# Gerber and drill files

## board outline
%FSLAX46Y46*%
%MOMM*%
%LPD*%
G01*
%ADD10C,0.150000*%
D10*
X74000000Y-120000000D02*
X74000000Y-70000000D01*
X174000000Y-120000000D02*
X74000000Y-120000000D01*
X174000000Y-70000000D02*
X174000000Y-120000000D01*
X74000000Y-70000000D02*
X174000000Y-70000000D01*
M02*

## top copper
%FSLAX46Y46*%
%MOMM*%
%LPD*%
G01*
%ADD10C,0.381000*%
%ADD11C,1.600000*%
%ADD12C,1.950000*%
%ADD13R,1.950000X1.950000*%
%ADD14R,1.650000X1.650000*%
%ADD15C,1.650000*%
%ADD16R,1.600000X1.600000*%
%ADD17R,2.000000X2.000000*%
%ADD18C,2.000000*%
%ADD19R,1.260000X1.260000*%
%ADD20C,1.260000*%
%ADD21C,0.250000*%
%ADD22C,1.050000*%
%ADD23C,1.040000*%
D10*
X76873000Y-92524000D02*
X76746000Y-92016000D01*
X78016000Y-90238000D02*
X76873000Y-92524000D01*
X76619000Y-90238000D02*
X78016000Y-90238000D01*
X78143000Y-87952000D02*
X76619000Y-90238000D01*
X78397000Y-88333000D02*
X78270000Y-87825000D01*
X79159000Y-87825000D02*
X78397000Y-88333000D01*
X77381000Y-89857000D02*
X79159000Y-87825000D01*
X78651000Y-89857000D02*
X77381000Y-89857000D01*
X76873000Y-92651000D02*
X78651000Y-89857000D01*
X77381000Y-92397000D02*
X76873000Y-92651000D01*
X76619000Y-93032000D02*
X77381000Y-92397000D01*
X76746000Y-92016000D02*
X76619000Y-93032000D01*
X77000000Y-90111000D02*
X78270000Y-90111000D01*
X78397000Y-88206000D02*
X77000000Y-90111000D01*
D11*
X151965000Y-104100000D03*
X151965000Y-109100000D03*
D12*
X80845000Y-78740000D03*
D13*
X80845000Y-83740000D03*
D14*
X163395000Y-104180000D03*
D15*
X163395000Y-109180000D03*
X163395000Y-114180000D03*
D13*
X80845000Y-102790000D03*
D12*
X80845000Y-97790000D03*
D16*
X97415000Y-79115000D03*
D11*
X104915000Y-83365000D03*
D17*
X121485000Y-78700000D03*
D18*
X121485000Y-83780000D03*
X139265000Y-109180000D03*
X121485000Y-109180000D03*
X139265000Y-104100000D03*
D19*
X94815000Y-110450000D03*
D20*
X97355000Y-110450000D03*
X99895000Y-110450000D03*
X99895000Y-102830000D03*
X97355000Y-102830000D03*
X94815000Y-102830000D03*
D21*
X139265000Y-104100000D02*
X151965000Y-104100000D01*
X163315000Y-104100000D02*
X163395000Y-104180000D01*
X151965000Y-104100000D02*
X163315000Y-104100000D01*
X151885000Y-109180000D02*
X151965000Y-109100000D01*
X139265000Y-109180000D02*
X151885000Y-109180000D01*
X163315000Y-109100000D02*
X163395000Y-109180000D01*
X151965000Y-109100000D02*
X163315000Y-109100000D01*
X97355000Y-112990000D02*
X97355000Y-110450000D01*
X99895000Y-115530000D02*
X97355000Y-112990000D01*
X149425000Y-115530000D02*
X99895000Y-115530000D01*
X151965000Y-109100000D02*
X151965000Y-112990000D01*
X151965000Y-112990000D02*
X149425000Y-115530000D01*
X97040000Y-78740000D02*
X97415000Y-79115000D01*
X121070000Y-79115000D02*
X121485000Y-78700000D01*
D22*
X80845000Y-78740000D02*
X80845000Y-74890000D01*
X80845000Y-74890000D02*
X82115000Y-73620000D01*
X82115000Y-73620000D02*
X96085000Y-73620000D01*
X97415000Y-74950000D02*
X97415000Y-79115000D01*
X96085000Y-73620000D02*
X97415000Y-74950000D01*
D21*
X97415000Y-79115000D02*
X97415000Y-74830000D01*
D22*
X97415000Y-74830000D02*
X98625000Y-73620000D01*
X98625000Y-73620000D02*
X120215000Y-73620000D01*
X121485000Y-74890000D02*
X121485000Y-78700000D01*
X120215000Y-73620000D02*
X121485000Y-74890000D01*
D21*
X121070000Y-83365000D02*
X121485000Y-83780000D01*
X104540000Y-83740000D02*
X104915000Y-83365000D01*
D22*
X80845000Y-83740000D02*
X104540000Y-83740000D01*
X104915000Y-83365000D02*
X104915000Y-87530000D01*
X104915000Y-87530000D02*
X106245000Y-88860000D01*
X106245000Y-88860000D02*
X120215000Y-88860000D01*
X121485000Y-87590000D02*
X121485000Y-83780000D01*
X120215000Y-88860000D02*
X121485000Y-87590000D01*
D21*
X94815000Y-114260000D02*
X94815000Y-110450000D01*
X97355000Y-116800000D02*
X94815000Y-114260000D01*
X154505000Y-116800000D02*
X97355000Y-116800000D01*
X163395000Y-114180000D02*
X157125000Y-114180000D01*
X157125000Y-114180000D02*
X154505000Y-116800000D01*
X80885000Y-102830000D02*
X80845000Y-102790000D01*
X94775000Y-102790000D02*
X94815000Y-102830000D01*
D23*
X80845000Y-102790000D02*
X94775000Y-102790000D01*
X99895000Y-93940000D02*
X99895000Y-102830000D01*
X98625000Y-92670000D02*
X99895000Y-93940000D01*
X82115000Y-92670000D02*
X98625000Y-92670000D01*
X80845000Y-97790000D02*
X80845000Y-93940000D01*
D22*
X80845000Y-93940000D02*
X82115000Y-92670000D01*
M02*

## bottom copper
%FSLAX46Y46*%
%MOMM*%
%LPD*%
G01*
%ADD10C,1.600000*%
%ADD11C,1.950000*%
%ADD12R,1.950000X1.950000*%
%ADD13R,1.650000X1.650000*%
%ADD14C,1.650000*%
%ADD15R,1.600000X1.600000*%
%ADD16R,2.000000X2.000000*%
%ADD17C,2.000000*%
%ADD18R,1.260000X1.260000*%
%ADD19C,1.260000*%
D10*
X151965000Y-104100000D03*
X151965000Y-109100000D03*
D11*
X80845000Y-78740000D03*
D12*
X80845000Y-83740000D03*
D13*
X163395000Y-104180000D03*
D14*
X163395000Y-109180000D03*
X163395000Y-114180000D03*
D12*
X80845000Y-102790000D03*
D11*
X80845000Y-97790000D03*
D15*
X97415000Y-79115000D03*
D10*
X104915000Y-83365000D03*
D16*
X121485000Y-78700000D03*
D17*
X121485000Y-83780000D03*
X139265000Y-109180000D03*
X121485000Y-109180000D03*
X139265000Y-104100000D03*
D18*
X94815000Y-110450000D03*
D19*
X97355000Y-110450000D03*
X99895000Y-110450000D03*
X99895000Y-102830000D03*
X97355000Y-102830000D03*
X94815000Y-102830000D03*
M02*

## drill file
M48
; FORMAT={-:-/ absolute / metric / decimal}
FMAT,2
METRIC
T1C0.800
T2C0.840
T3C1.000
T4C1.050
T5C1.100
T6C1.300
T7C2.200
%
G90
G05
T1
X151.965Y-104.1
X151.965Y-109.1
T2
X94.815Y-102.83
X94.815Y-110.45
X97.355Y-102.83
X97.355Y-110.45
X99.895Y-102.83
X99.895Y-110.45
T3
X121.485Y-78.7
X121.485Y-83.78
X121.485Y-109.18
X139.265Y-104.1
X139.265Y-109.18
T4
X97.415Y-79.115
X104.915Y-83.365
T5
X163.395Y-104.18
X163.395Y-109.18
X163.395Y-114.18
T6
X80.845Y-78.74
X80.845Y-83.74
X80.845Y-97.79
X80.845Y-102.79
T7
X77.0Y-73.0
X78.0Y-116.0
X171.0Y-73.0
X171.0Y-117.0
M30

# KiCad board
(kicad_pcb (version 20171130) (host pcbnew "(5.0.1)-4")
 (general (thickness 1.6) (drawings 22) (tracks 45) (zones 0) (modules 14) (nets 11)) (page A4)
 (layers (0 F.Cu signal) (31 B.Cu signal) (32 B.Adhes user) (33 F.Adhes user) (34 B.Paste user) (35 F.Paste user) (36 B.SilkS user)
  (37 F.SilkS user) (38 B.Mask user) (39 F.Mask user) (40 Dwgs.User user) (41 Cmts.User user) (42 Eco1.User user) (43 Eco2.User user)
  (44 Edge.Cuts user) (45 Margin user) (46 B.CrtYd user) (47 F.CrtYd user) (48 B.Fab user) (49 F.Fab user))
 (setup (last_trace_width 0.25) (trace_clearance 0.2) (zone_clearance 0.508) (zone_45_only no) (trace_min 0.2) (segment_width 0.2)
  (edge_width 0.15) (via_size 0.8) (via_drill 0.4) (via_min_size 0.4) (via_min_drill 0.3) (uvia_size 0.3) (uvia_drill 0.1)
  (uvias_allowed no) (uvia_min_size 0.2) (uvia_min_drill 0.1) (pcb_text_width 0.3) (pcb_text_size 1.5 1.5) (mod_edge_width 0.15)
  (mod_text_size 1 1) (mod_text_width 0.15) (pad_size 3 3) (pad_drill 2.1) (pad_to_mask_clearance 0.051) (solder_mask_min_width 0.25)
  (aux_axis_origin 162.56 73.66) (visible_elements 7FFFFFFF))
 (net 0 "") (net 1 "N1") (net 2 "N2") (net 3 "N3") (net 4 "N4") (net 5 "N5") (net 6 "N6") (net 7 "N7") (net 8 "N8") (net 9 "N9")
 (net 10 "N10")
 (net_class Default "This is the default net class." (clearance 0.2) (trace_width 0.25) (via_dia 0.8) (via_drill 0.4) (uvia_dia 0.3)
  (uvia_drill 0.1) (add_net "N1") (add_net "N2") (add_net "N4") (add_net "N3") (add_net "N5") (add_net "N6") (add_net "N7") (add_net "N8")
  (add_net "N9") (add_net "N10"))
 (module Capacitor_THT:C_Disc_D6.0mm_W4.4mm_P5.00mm (layer F.Cu) (at 151.965 104.1 270)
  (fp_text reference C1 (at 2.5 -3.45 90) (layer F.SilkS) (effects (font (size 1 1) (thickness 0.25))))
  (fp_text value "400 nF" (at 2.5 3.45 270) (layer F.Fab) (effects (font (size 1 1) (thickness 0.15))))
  (pad 1 thru_hole circle (at 0 0 270) (size 1.6 1.6) (drill 0.8) (layers *.Cu *.Mask) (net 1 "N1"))
  (pad 2 thru_hole circle (at 5 0 270) (size 1.6 1.6) (drill 0.8) (layers *.Cu *.Mask) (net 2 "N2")))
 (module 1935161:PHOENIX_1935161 (layer F.Cu) (at 80.845 81.24 90)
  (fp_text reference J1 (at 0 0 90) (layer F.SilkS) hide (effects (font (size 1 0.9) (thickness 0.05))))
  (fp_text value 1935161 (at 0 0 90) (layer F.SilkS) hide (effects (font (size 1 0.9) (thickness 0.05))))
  (pad 2 thru_hole circle (at 2.5 0 90) (size 1.95 1.95) (drill 1.3) (layers *.Cu *.Mask) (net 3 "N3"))
  (pad 1 thru_hole rect (at -2.5 0 90) (size 1.95 1.95) (drill 1.3) (layers *.Cu *.Mask) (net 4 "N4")))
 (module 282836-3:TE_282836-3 (layer F.Cu) (at 163.395 109.18 270)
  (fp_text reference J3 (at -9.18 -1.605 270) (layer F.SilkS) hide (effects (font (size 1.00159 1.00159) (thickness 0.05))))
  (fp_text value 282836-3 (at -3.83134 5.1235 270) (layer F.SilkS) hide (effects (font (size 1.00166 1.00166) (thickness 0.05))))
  (pad 1 thru_hole rect (at -5 0 270) (size 1.65 1.65) (drill 1.1) (layers *.Cu *.Mask) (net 1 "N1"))
  (pad 2 thru_hole circle (at 0 0 270) (size 1.65 1.65) (drill 1.1) (layers *.Cu *.Mask) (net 2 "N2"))
  (pad 3 thru_hole circle (at 5 0 270) (size 1.65 1.65) (drill 1.1) (layers *.Cu *.Mask) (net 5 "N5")))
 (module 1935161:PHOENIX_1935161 (layer F.Cu) (at 80.845 100.29 90)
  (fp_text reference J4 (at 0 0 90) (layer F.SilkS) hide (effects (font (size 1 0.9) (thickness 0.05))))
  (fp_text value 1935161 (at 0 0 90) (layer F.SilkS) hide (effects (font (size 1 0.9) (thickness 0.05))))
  (pad 1 thru_hole rect (at -2.5 0 90) (size 1.95 1.95) (drill 1.3) (layers *.Cu *.Mask) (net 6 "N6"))
  (pad 2 thru_hole circle (at 2.5 0 90) (size 1.95 1.95) (drill 1.3) (layers *.Cu *.Mask) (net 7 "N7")))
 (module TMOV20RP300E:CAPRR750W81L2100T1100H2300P (layer F.Cu) (at 101.165 81.24)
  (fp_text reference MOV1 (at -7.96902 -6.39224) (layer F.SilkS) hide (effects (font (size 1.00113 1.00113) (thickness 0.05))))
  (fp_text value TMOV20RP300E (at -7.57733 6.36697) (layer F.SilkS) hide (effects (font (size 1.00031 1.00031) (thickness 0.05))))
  (pad 1 thru_hole rect (at -3.75 -2.125) (size 1.6 1.6) (drill 1.05) (layers *.Cu *.Mask) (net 3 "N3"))
  (pad 2 thru_hole circle (at 3.75 2.125) (size 1.6 1.6) (drill 1.05) (layers *.Cu *.Mask) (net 4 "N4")))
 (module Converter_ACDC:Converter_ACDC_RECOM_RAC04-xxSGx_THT (layer F.Cu) (at 121.485 78.7)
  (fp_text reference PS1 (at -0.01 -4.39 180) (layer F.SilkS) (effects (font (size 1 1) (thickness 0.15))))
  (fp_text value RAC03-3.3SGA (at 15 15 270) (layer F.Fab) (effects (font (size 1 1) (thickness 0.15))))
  (pad 1 thru_hole rect (at 0 0 90) (size 2 2) (drill 1) (layers *.Cu *.Mask) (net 3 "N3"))
  (pad 2 thru_hole circle (at 0 5.08 90) (size 2 2) (drill 1) (layers *.Cu *.Mask) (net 4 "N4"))
  (pad 4 thru_hole circle (at 17.78 30.48 90) (size 2 2) (drill 1) (layers *.Cu *.Mask) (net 2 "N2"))
  (pad 3 thru_hole circle (at 0 30.48 180) (size 2 2) (drill 1) (layers *.Cu *.Mask) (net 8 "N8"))
  (pad 5 thru_hole circle (at 17.78 25.4 90) (size 2 2) (drill 1) (layers *.Cu *.Mask) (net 1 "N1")))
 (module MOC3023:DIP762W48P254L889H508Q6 (layer F.Cu) (at 97.355 106.64 90)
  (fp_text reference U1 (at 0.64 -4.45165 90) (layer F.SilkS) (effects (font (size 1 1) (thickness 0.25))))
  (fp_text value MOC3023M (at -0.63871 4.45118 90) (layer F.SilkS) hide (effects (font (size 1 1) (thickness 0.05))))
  (pad 1 thru_hole rect (at -3.81 -2.54 90) (size 1.26 1.26) (drill 0.84) (layers *.Cu *.Mask) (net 5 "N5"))
  (pad 2 thru_hole circle (at -3.81 0 90) (size 1.26 1.26) (drill 0.84) (layers *.Cu *.Mask) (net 2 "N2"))
  (pad 3 thru_hole circle (at -3.81 2.54 90) (size 1.26 1.26) (drill 0.84) (layers *.Cu *.Mask) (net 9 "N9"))
  (pad 4 thru_hole circle (at 3.81 2.54 90) (size 1.26 1.26) (drill 0.84) (layers *.Cu *.Mask) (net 7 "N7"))
  (pad 5 thru_hole circle (at 3.81 0 90) (size 1.26 1.26) (drill 0.84) (layers *.Cu *.Mask) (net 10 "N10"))
  (pad 6 thru_hole circle (at 3.81 -2.54 90) (size 1.26 1.26) (drill 0.84) (layers *.Cu *.Mask) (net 6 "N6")))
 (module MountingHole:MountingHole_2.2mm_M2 (layer F.Cu) (at 171 73)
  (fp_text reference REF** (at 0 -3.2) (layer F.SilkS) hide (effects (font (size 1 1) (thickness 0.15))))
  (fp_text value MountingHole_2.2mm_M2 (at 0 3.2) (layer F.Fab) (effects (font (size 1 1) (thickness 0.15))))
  (pad 1 np_thru_hole circle (at 0 0) (size 2.2 2.2) (drill 2.2) (layers *.Cu *.Mask)))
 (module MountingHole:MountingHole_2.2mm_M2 (layer F.Cu) (at 78 116)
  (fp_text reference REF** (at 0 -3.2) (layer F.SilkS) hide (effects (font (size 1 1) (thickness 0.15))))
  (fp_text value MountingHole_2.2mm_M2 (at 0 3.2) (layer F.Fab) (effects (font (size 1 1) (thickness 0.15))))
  (pad 1 np_thru_hole circle (at 0 0) (size 2.2 2.2) (drill 2.2) (layers *.Cu *.Mask)))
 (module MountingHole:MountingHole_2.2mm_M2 (layer F.Cu) (at 171 117)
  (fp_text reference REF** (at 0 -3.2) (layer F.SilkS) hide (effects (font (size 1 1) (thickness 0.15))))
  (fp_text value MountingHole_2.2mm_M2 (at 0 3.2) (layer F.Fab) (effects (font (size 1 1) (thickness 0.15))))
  (pad 1 np_thru_hole circle (at 0 0) (size 2.2 2.2) (drill 2.2) (layers *.Cu *.Mask)))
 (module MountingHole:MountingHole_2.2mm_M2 (layer F.Cu) (at 77 73)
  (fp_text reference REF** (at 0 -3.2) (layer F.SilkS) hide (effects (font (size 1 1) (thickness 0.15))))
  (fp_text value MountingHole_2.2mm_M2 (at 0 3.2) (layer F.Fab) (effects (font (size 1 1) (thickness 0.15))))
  (pad 1 np_thru_hole circle (at 0 0) (size 2.2 2.2) (drill 2.2) (layers *.Cu *.Mask)))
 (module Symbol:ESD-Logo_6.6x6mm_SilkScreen (layer F.Cu) (at 110 96)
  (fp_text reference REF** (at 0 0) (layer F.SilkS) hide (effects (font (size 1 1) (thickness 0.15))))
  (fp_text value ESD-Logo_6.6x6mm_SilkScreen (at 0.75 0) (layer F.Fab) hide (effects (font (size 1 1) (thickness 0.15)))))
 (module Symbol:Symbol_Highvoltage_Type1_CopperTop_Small (layer F.Cu) (at 77 91)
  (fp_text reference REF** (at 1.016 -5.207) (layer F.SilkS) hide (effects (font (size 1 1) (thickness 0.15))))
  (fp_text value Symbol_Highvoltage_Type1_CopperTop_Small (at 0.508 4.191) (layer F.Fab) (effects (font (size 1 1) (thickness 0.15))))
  (fp_line (start -0.127 1.524) (end -0.254 1.016) (layer F.Cu) (width 0.381))
  (fp_line (start 1.016 -0.762) (end -0.127 1.524) (layer F.Cu) (width 0.381))
  (fp_line (start -0.381 -0.762) (end 1.016 -0.762) (layer F.Cu) (width 0.381))
  (fp_line (start 1.143 -3.048) (end -0.381 -0.762) (layer F.Cu) (width 0.381))
  (fp_line (start 1.397 -2.667) (end 1.27 -3.175) (layer F.Cu) (width 0.381))
  (fp_line (start 2.159 -3.175) (end 1.397 -2.667) (layer F.Cu) (width 0.381))
  (fp_line (start 0.381 -1.143) (end 2.159 -3.175) (layer F.Cu) (width 0.381))
  (fp_line (start 1.651 -1.143) (end 0.381 -1.143) (layer F.Cu) (width 0.381))
  (fp_line (start -0.127 1.651) (end 1.651 -1.143) (layer F.Cu) (width 0.381))
  (fp_line (start 0.381 1.397) (end -0.127 1.651) (layer F.Cu) (width 0.381))
  (fp_line (start -0.381 2.032) (end 0.381 1.397) (layer F.Cu) (width 0.381))
  (fp_line (start -0.254 1.016) (end -0.381 2.032) (layer F.Cu) (width 0.381))
  (fp_line (start 0 -0.889) (end 1.27 -0.889) (layer F.Cu) (width 0.381))
  (fp_line (start 1.397 -2.794) (end 0 -0.889) (layer F.Cu) (width 0.381)))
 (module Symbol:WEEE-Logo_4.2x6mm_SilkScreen (layer F.Cu) (at 86 112)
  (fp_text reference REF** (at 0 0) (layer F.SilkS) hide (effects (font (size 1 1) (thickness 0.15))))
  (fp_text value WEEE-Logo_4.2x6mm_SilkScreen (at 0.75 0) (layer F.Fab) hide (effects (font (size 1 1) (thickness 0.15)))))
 (gr_line (start 74 120) (end 74 70) (layer Edge.Cuts) (width 0.15))
 (gr_line (start 174 120) (end 74 120) (layer Edge.Cuts) (width 0.15))
 (gr_line (start 174 70) (end 174 120) (layer Edge.Cuts) (width 0.15))
 (gr_line (start 74 70) (end 174 70) (layer Edge.Cuts) (width 0.15))
 (segment (start 139.265 104.1) (end 151.965 104.1) (width 0.25) (layer F.Cu) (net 1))
 (segment (start 163.315 104.1) (end 163.395 104.18) (width 0.25) (layer F.Cu) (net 1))
 (segment (start 151.965 104.1) (end 163.315 104.1) (width 0.25) (layer F.Cu) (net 1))
 (segment (start 151.885 109.18) (end 151.965 109.1) (width 0.25) (layer F.Cu) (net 2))
 (segment (start 139.265 109.18) (end 151.885 109.18) (width 0.25) (layer F.Cu) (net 2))
 (segment (start 163.315 109.1) (end 163.395 109.18) (width 0.25) (layer F.Cu) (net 2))
 (segment (start 151.965 109.1) (end 163.315 109.1) (width 0.25) (layer F.Cu) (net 2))
 (segment (start 97.355 112.99) (end 97.355 110.45) (width 0.25) (layer F.Cu) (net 2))
 (segment (start 99.895 115.53) (end 97.355 112.99) (width 0.25) (layer F.Cu) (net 2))
 (segment (start 149.425 115.53) (end 99.895 115.53) (width 0.25) (layer F.Cu) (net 2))
 (segment (start 151.965 109.1) (end 151.965 112.99) (width 0.25) (layer F.Cu) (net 2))
 (segment (start 151.965 112.99) (end 149.425 115.53) (width 0.25) (layer F.Cu) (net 2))
 (segment (start 97.04 78.74) (end 97.415 79.115) (width 0.25) (layer F.Cu) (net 3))
 (segment (start 121.07 79.115) (end 121.485 78.7) (width 0.25) (layer F.Cu) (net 3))
 (segment (start 80.845 78.74) (end 80.845 74.89) (width 1.05) (layer F.Cu) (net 3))
 (segment (start 80.845 74.89) (end 82.115 73.62) (width 1.05) (layer F.Cu) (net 3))
 (segment (start 82.115 73.62) (end 96.085 73.62) (width 1.05) (layer F.Cu) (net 3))
 (segment (start 97.415 74.95) (end 97.415 79.115) (width 1.05) (layer F.Cu) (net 3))
 (segment (start 96.085 73.62) (end 97.415 74.95) (width 1.05) (layer F.Cu) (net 3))
 (segment (start 97.415 79.115) (end 97.415 74.83) (width 0.25) (layer F.Cu) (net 3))
 (segment (start 97.415 74.83) (end 98.625 73.62) (width 1.05) (layer F.Cu) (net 3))
 (segment (start 98.625 73.62) (end 120.215 73.62) (width 1.05) (layer F.Cu) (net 3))
 (segment (start 121.485 74.89) (end 121.485 78.7) (width 1.05) (layer F.Cu) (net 3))
 (segment (start 120.215 73.62) (end 121.485 74.89) (width 1.05) (layer F.Cu) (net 3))
 (segment (start 121.07 83.365) (end 121.485 83.78) (width 0.25) (layer F.Cu) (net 4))
 (segment (start 104.54 83.74) (end 104.915 83.365) (width 0.25) (layer F.Cu) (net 4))
 (segment (start 80.845 83.74) (end 104.54 83.74) (width 1.05) (layer F.Cu) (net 4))
 (segment (start 104.915 83.365) (end 104.915 87.53) (width 1.05) (layer F.Cu) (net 4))
 (segment (start 104.915 87.53) (end 106.245 88.86) (width 1.05) (layer F.Cu) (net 4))
 (segment (start 106.245 88.86) (end 120.215 88.86) (width 1.05) (layer F.Cu) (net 4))
 (segment (start 121.485 87.59) (end 121.485 83.78) (width 1.05) (layer F.Cu) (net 4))
 (segment (start 120.215 88.86) (end 121.485 87.59) (width 1.05) (layer F.Cu) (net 4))
 (segment (start 94.815 114.26) (end 94.815 110.45) (width 0.25) (layer F.Cu) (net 5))
 (segment (start 97.355 116.8) (end 94.815 114.26) (width 0.25) (layer F.Cu) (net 5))
 (segment (start 154.505 116.8) (end 97.355 116.8) (width 0.25) (layer F.Cu) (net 5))
 (segment (start 163.395 114.18) (end 157.125 114.18) (width 0.25) (layer F.Cu) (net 5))
 (segment (start 157.125 114.18) (end 154.505 116.8) (width 0.25) (layer F.Cu) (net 5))
 (segment (start 80.885 102.83) (end 80.845 102.79) (width 0.25) (layer F.Cu) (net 6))
 (segment (start 94.775 102.79) (end 94.815 102.83) (width 0.25) (layer F.Cu) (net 6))
 (segment (start 80.845 102.79) (end 94.775 102.79) (width 1.04) (layer F.Cu) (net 6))
 (segment (start 99.895 93.94) (end 99.895 102.83) (width 1.04) (layer F.Cu) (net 7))
 (segment (start 98.625 92.67) (end 99.895 93.94) (width 1.04) (layer F.Cu) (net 7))
 (segment (start 82.115 92.67) (end 98.625 92.67) (width 1.04) (layer F.Cu) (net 7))
 (segment (start 80.845 97.79) (end 80.845 93.94) (width 1.04) (layer F.Cu) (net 7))
 (segment (start 80.845 93.94) (end 82.115 92.67) (width 1.05) (layer F.Cu) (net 7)))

